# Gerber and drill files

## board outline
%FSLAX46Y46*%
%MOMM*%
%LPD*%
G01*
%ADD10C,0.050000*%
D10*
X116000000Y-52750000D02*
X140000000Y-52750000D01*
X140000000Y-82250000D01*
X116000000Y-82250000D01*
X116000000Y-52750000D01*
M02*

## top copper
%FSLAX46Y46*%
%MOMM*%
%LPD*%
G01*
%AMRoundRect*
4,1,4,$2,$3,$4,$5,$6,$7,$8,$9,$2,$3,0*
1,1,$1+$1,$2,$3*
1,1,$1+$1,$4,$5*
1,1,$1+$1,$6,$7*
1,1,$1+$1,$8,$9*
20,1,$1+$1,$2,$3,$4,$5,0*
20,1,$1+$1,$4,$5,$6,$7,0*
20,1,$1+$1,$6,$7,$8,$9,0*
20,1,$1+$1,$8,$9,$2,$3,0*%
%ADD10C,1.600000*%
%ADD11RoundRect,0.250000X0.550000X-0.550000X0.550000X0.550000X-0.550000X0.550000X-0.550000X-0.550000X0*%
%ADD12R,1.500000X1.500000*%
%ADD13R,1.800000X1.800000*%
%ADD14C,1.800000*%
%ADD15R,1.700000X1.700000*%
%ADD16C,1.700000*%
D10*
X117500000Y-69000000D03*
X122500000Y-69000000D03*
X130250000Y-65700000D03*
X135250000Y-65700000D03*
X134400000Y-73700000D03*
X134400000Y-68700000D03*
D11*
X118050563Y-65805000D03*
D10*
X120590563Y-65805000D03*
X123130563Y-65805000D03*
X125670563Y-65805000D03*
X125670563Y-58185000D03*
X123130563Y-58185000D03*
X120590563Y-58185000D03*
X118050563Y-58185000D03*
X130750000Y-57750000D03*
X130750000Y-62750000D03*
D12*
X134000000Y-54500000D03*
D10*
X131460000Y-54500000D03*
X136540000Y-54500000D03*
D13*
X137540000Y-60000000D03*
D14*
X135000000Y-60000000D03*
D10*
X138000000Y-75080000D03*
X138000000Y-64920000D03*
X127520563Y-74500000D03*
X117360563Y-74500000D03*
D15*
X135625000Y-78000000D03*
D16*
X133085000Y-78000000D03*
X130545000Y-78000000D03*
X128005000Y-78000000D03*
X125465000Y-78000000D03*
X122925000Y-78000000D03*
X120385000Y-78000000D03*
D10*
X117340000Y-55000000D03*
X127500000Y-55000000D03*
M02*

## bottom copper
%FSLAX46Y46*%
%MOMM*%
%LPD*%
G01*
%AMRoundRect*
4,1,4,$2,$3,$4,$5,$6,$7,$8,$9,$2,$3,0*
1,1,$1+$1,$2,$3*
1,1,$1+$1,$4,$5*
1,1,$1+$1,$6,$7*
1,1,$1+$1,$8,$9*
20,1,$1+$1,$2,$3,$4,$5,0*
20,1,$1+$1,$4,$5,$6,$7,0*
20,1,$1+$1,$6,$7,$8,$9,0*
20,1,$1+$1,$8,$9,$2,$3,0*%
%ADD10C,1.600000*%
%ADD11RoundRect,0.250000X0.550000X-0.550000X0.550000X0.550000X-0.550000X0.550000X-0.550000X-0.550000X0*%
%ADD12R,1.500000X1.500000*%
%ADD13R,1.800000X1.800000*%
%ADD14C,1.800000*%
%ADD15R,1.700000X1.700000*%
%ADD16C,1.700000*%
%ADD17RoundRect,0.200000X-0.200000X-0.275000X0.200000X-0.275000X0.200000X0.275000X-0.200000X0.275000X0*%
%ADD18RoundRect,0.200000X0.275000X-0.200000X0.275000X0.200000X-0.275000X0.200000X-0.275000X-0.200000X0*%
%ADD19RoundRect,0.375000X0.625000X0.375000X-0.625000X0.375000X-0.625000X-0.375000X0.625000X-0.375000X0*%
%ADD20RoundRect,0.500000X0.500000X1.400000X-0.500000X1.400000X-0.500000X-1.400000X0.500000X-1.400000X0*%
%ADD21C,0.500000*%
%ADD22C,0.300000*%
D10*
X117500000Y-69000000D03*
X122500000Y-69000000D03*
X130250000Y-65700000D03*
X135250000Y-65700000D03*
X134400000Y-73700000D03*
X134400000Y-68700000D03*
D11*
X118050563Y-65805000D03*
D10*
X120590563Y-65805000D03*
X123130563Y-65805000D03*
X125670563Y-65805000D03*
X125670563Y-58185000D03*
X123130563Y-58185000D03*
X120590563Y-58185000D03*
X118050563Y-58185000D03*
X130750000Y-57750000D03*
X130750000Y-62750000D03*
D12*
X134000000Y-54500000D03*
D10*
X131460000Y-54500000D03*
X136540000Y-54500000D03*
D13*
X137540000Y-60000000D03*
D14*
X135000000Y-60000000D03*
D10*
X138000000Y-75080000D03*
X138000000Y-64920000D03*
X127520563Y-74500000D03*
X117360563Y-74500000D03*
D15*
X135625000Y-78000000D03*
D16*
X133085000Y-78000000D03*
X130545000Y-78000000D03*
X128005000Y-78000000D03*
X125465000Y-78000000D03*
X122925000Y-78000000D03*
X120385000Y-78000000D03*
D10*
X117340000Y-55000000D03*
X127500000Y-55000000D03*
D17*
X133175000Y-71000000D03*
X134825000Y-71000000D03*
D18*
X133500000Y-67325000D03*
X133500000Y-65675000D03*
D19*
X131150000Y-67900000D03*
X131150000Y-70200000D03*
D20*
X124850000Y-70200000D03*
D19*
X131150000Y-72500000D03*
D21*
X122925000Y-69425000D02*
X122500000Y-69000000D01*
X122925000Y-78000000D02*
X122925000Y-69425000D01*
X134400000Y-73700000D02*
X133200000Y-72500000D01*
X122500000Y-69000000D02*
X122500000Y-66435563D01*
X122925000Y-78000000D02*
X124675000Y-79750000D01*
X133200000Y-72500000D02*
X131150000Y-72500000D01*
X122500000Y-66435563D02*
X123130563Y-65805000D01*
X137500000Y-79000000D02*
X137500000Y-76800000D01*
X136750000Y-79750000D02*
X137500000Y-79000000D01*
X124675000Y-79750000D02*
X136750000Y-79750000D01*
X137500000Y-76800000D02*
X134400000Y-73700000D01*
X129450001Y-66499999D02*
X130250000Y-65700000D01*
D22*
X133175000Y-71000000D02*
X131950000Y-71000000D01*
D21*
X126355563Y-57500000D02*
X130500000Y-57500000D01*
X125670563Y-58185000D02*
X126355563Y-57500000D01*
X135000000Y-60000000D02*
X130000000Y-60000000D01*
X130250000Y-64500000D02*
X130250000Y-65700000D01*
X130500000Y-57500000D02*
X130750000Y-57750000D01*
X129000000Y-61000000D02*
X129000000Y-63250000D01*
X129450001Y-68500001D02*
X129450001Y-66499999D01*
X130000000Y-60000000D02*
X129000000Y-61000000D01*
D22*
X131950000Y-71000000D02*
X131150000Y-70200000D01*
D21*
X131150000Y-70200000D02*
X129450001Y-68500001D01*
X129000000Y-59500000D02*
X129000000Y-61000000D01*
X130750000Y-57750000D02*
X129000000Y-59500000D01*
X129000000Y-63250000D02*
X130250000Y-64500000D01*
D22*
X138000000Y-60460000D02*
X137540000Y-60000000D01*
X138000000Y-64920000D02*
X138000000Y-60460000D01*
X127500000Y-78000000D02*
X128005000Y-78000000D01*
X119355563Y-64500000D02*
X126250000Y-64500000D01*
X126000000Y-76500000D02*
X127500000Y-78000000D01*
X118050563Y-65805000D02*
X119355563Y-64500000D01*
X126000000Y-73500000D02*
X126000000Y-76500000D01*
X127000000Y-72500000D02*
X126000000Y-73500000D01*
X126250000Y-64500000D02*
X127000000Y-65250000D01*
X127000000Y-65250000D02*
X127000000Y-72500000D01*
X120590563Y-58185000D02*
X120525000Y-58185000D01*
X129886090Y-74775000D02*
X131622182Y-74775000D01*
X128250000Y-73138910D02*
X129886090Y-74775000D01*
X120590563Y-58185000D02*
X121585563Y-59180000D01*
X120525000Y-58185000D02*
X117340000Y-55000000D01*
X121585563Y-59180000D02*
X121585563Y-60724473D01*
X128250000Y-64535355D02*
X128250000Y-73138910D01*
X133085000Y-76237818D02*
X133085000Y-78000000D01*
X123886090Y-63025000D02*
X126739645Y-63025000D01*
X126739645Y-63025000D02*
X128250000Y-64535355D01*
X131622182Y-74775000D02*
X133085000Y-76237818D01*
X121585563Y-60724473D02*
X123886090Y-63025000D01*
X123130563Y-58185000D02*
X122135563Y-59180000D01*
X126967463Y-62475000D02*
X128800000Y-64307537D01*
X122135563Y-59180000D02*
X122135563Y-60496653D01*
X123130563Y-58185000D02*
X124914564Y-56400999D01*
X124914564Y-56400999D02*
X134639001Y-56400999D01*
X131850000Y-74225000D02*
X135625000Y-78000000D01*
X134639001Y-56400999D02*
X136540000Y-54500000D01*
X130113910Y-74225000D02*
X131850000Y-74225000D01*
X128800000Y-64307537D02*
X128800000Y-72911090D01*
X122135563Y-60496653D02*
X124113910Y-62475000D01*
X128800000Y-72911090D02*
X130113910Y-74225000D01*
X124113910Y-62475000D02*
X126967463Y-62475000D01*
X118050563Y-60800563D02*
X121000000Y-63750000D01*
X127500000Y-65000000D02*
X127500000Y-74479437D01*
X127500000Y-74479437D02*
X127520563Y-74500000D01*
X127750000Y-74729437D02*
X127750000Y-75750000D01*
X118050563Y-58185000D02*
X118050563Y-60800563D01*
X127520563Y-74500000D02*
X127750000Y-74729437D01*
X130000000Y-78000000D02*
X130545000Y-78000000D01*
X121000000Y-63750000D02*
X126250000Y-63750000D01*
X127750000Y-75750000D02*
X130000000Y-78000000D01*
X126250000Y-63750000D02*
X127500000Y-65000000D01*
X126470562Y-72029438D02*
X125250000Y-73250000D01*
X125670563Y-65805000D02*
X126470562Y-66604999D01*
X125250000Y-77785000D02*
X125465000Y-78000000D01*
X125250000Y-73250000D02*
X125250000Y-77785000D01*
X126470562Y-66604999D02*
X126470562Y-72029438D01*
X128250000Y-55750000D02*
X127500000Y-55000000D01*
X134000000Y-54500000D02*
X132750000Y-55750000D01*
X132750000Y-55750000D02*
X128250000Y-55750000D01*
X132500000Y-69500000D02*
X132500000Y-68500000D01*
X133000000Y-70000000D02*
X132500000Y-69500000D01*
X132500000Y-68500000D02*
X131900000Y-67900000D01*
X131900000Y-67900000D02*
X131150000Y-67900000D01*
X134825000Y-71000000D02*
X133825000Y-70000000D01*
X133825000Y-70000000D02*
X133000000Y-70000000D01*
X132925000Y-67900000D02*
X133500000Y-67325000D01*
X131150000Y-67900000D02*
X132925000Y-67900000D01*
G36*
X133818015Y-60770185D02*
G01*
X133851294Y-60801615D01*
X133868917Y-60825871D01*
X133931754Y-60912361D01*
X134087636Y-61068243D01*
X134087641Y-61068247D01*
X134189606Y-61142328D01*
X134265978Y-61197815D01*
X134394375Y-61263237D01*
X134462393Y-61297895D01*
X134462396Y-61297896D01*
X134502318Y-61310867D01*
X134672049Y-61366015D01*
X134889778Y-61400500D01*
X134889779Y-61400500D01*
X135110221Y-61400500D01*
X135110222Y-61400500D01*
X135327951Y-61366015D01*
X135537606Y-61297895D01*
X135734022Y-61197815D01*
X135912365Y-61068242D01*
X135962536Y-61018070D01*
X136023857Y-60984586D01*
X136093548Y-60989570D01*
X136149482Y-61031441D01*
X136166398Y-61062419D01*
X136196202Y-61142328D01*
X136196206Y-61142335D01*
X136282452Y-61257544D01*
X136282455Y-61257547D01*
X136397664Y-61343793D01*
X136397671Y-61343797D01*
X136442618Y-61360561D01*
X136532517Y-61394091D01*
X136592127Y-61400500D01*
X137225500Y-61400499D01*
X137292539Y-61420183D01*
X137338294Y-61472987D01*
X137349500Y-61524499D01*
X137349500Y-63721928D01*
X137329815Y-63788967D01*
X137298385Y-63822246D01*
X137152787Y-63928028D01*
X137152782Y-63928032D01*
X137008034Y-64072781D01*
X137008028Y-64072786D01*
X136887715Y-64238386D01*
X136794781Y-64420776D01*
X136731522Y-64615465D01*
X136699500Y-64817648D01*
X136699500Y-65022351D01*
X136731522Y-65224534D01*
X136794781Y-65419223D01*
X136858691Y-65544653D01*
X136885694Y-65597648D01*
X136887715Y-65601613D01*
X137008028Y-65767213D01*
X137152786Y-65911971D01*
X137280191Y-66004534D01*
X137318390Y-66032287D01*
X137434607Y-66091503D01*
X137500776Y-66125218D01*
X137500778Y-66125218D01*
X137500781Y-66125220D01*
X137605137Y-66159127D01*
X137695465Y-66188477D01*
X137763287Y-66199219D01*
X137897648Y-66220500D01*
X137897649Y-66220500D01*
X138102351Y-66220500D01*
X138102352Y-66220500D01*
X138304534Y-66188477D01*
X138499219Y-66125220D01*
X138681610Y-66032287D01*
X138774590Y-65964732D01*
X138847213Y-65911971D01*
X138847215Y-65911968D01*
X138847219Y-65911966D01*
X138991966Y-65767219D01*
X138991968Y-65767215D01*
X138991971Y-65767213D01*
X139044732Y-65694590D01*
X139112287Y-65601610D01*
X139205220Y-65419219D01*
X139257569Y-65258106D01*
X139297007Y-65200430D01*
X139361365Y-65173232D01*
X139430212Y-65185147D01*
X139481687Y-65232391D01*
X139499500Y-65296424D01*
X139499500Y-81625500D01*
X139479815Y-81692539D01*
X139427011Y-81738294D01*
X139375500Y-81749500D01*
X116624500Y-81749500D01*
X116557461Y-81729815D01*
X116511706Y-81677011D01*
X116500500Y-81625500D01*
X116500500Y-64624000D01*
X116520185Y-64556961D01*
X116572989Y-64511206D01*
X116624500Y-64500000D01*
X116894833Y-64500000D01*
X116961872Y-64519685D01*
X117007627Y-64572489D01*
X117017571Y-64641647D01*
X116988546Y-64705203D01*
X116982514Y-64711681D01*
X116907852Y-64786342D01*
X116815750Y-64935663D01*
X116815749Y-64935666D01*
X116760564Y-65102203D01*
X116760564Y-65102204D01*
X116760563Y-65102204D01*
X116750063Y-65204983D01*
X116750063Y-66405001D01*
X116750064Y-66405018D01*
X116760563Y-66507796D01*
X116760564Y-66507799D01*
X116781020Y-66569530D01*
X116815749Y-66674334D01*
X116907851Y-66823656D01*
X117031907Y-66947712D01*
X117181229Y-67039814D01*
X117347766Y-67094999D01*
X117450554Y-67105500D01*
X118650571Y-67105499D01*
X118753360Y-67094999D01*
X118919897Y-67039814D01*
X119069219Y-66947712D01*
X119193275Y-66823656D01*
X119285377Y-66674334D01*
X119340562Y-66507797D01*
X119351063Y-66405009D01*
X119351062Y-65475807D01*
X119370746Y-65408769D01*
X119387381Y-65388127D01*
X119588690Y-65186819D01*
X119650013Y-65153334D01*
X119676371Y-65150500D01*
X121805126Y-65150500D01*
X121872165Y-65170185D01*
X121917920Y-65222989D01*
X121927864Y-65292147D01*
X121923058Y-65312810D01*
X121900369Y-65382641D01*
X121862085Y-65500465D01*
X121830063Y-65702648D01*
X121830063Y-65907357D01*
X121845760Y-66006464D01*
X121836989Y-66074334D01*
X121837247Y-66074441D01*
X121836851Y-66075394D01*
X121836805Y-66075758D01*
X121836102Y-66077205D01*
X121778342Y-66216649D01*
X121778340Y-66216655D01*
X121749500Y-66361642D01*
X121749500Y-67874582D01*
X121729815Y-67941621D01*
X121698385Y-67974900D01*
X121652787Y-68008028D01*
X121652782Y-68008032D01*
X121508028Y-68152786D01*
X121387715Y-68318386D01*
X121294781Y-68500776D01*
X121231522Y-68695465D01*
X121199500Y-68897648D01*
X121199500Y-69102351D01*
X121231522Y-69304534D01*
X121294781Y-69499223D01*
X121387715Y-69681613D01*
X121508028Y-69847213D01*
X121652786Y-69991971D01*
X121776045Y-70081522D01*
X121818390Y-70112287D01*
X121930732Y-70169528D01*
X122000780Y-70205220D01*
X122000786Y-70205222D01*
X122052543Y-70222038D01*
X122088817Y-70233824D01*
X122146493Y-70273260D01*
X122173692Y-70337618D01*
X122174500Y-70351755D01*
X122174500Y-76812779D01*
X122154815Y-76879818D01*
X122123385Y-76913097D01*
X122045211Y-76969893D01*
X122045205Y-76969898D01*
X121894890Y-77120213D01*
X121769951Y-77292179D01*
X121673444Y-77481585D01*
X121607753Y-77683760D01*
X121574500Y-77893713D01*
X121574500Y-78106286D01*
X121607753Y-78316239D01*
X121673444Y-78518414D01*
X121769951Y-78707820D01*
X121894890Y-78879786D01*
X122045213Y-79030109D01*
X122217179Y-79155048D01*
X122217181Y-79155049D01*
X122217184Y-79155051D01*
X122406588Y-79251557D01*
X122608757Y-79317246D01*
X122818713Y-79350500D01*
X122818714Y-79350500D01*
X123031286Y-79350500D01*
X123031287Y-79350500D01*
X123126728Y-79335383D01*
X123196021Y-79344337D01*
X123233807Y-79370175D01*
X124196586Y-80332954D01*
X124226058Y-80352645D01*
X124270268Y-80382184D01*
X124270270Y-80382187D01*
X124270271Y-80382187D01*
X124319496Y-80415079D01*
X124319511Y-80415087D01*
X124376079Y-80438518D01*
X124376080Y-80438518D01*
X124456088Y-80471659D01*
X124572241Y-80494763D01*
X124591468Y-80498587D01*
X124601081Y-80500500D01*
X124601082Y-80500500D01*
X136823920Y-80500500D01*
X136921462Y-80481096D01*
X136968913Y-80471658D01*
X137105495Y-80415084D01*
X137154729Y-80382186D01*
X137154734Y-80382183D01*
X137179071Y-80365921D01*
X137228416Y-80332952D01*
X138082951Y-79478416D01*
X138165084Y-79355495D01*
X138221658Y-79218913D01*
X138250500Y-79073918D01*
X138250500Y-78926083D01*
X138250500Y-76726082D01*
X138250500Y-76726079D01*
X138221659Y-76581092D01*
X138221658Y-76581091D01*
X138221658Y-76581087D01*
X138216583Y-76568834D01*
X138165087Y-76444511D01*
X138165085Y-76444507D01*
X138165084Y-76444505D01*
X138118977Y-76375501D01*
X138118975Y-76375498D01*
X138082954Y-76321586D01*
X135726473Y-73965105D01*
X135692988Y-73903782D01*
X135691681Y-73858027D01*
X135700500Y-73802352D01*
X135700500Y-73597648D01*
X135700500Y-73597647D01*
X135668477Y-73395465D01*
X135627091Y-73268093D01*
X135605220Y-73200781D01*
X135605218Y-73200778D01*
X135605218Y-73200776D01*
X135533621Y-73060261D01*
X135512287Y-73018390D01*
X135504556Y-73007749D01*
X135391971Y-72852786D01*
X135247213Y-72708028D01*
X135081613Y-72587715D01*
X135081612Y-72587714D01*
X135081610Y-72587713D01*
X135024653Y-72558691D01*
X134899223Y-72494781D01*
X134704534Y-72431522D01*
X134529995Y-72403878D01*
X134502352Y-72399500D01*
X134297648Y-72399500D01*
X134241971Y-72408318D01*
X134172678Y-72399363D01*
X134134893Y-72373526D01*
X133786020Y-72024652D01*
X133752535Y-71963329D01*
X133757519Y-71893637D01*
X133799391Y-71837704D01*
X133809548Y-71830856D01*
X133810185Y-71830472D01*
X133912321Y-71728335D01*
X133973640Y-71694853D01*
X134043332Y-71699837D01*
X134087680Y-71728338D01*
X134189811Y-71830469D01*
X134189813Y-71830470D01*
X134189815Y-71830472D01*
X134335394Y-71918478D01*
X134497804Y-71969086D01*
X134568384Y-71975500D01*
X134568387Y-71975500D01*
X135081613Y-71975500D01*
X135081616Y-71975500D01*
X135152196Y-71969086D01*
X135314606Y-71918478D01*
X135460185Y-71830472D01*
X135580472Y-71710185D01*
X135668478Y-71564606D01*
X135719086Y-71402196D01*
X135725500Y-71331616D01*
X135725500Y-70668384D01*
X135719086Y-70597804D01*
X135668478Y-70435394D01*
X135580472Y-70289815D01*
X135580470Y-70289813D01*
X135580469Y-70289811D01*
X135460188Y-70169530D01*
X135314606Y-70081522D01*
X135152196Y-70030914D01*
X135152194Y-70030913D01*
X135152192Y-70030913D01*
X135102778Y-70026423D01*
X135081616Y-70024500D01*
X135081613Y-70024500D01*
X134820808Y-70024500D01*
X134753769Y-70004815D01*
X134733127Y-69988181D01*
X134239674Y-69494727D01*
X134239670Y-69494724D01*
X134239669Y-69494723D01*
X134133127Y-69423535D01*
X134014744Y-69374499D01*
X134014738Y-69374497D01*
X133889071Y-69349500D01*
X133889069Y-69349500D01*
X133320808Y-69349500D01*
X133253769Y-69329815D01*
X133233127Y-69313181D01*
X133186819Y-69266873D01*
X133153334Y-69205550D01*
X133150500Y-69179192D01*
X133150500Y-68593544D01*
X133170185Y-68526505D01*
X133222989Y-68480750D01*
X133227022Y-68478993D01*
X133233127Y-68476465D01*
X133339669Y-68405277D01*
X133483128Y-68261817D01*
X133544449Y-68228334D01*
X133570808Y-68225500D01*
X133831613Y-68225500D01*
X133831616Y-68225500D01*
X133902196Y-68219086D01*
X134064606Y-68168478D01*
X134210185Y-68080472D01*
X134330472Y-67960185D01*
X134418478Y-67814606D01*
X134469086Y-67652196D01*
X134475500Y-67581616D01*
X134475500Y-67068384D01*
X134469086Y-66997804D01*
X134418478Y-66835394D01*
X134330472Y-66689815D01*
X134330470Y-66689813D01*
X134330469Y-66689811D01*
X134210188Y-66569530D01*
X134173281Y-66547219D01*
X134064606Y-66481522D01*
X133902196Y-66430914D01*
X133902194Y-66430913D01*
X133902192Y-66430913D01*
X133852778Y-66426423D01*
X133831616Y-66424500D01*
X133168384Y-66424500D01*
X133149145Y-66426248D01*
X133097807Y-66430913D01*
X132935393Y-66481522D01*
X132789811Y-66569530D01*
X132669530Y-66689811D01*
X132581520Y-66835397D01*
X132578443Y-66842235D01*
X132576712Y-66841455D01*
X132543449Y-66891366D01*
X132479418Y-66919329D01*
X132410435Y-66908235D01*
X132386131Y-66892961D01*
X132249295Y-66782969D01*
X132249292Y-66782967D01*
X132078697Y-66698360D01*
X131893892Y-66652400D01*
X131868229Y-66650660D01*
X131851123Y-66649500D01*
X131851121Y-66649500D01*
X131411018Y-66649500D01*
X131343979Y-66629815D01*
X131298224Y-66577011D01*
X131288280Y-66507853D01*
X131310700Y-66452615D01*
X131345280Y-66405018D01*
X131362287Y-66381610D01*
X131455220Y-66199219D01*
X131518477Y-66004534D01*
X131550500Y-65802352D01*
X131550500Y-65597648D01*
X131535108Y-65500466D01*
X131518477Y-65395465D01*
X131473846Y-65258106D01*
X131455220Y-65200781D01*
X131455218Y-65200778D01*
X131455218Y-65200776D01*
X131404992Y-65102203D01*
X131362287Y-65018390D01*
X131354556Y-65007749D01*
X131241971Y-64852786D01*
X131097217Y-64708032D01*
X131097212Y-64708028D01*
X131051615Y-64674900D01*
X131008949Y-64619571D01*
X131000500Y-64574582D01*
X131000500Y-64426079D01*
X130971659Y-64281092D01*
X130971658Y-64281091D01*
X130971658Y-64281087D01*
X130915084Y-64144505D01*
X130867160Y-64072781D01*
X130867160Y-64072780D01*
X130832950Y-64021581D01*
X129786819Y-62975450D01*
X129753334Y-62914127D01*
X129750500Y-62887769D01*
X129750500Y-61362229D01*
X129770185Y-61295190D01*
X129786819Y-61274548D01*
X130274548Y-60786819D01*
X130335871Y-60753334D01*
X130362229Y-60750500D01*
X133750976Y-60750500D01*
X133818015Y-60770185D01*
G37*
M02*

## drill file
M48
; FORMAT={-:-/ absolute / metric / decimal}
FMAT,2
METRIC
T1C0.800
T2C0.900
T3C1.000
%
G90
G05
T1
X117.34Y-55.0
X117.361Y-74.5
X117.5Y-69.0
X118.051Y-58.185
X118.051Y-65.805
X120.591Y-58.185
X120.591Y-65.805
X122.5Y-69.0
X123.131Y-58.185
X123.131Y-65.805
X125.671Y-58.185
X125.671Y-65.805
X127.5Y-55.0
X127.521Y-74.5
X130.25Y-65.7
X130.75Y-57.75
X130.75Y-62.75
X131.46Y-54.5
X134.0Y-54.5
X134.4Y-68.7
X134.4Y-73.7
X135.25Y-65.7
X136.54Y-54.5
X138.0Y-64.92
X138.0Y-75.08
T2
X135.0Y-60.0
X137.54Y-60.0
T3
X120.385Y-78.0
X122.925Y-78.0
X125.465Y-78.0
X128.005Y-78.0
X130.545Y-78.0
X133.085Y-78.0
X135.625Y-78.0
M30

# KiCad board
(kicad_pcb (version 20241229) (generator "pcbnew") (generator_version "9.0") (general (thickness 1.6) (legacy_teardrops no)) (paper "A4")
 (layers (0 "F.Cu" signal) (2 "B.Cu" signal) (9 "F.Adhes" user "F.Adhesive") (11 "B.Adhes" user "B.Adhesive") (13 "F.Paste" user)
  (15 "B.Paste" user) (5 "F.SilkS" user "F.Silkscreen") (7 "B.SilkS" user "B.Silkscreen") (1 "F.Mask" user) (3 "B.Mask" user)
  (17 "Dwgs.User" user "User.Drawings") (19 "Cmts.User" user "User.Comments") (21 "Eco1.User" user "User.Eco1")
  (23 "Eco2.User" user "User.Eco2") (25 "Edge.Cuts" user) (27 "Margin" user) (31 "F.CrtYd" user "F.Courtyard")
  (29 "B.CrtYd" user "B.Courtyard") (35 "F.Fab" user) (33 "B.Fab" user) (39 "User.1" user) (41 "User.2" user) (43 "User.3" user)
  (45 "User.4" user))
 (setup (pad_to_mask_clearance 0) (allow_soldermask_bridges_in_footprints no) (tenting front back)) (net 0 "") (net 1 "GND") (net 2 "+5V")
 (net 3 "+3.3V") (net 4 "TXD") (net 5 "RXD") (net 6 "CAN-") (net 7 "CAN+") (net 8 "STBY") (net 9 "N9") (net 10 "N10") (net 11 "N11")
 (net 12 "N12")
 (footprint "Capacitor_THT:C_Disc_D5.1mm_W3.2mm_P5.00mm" (layer "F.Cu") (at 117.5 69)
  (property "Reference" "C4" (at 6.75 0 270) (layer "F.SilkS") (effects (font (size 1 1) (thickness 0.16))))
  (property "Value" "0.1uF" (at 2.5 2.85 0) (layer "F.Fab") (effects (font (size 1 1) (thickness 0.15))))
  (pad "1" thru_hole circle (at 0 0) (size 1.6 1.6) (drill 0.8) (layers "*.Cu" "*.Mask") (remove_unused_layers no) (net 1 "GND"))
  (pad "2" thru_hole circle (at 5 0) (size 1.6 1.6) (drill 0.8) (layers "*.Cu" "*.Mask") (remove_unused_layers no) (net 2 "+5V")))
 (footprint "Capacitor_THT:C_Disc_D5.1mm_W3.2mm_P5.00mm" (layer "F.Cu") (at 130.25 65.7)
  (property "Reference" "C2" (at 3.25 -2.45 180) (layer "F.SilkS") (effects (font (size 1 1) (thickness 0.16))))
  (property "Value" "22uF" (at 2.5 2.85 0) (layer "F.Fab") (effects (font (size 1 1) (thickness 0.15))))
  (pad "1" thru_hole circle (at 0 0) (size 1.6 1.6) (drill 0.8) (layers "*.Cu" "*.Mask") (remove_unused_layers no) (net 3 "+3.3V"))
  (pad "2" thru_hole circle (at 5 0) (size 1.6 1.6) (drill 0.8) (layers "*.Cu" "*.Mask") (remove_unused_layers no) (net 1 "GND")))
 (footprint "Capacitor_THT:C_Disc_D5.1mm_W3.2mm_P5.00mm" (layer "F.Cu") (at 134.4 73.7 90)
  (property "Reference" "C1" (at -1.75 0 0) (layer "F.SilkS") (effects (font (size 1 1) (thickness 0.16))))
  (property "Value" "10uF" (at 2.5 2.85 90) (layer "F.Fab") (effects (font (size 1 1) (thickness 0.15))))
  (pad "1" thru_hole circle (at 0 0 90) (size 1.6 1.6) (drill 0.8) (layers "*.Cu" "*.Mask") (remove_unused_layers no) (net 2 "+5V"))
  (pad "2" thru_hole circle (at 5 0 90) (size 1.6 1.6) (drill 0.8) (layers "*.Cu" "*.Mask") (remove_unused_layers no) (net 1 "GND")))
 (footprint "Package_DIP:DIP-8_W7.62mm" (layer "F.Cu") (at 118.050563 65.805 90)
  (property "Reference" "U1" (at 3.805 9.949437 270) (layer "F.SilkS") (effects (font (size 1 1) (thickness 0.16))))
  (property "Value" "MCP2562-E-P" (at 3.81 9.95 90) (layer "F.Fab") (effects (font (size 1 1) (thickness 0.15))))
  (pad "1" thru_hole roundrect (at 0 0 90) (size 1.6 1.6) (drill 0.8) (layers "*.Cu" "*.Mask") (remove_unused_layers no)
   (roundrect_rratio 0.15625) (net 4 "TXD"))
  (pad "2" thru_hole circle (at 0 2.54 90) (size 1.6 1.6) (drill 0.8) (layers "*.Cu" "*.Mask") (remove_unused_layers no) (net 1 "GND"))
  (pad "3" thru_hole circle (at 0 5.08 90) (size 1.6 1.6) (drill 0.8) (layers "*.Cu" "*.Mask") (remove_unused_layers no) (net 2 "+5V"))
  (pad "4" thru_hole circle (at 0 7.62 90) (size 1.6 1.6) (drill 0.8) (layers "*.Cu" "*.Mask") (remove_unused_layers no) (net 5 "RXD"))
  (pad "5" thru_hole circle (at 7.62 7.62 90) (size 1.6 1.6) (drill 0.8) (layers "*.Cu" "*.Mask") (remove_unused_layers no) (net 3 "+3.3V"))
  (pad "6" thru_hole circle (at 7.62 5.08 90) (size 1.6 1.6) (drill 0.8) (layers "*.Cu" "*.Mask") (remove_unused_layers no) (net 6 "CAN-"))
  (pad "7" thru_hole circle (at 7.62 2.54 90) (size 1.6 1.6) (drill 0.8) (layers "*.Cu" "*.Mask") (remove_unused_layers no) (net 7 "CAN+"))
  (pad "8" thru_hole circle (at 7.62 0 90) (size 1.6 1.6) (drill 0.8) (layers "*.Cu" "*.Mask") (remove_unused_layers no) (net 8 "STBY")))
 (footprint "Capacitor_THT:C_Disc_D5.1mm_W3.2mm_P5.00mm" (layer "F.Cu") (at 130.75 57.75 -90)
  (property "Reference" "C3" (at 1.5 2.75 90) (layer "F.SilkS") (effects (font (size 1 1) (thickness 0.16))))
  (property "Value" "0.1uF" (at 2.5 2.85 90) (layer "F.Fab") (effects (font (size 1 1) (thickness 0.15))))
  (pad "1" thru_hole circle (at 0 0 270) (size 1.6 1.6) (drill 0.8) (layers "*.Cu" "*.Mask") (remove_unused_layers no) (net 3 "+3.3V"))
  (pad "2" thru_hole circle (at 5 0 270) (size 1.6 1.6) (drill 0.8) (layers "*.Cu" "*.Mask") (remove_unused_layers no) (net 1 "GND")))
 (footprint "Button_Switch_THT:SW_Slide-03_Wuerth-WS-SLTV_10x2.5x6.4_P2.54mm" (layer "F.Cu") (at 134 54.5)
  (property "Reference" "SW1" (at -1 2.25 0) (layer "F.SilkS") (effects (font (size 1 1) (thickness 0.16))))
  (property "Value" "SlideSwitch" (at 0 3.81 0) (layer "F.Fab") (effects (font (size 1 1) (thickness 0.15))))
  (pad "1" thru_hole rect (at 0 0) (size 1.5 1.5) (drill 0.8) (layers "*.Cu" "*.Mask") (remove_unused_layers no) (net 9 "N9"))
  (pad "2" thru_hole circle (at -2.54 0) (size 1.6 1.6) (drill 0.8) (layers "*.Cu" "*.Mask") (remove_unused_layers no) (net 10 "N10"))
  (pad "3" thru_hole circle (at 2.54 0) (size 1.6 1.6) (drill 0.8) (layers "*.Cu" "*.Mask") (remove_unused_layers no) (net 6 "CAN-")))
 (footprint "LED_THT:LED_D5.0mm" (layer "F.Cu") (at 137.54 60 180)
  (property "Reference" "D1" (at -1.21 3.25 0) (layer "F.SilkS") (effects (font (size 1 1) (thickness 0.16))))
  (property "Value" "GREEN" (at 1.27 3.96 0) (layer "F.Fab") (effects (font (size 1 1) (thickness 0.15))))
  (pad "1" thru_hole rect (at 0 0 180) (size 1.8 1.8) (drill 0.9) (layers "*.Cu" "*.Mask") (remove_unused_layers no) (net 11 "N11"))
  (pad "2" thru_hole circle (at 2.54 0 180) (size 1.8 1.8) (drill 0.9) (layers "*.Cu" "*.Mask") (remove_unused_layers no) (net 3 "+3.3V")))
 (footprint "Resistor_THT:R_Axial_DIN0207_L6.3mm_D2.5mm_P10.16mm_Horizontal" (layer "F.Cu") (at 138 75.08 90)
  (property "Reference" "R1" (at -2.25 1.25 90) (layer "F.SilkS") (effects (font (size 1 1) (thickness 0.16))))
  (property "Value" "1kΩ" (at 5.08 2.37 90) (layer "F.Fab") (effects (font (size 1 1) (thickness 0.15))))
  (pad "1" thru_hole circle (at 0 0 90) (size 1.6 1.6) (drill 0.8) (layers "*.Cu" "*.Mask") (remove_unused_layers no) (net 1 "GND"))
  (pad "2" thru_hole circle (at 10.16 0 90) (size 1.6 1.6) (drill 0.8) (layers "*.Cu" "*.Mask") (remove_unused_layers no) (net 11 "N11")))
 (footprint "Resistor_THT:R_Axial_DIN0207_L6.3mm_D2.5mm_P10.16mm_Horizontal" (layer "F.Cu") (at 127.520563 74.5 180)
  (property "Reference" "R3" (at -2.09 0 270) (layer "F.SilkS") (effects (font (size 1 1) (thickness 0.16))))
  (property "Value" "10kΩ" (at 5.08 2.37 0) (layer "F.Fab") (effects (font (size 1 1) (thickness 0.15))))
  (pad "1" thru_hole circle (at 0 0 180) (size 1.6 1.6) (drill 0.8) (layers "*.Cu" "*.Mask") (remove_unused_layers no) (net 8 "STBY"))
  (pad "2" thru_hole circle (at 10.16 0 180) (size 1.6 1.6) (drill 0.8) (layers "*.Cu" "*.Mask") (remove_unused_layers no) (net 1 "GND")))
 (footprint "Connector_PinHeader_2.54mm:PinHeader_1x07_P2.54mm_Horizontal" (layer "F.Cu") (at 135.625 78 -90)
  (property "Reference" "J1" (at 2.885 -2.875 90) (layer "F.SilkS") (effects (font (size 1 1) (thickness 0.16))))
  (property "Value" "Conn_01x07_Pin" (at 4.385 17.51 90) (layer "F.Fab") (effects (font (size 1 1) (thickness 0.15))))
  (pad "1" thru_hole rect (at 0 0 270) (size 1.7 1.7) (drill 1) (layers "*.Cu" "*.Mask") (remove_unused_layers no) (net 6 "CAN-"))
  (pad "2" thru_hole circle (at 0 2.54 270) (size 1.7 1.7) (drill 1) (layers "*.Cu" "*.Mask") (remove_unused_layers no) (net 7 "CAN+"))
  (pad "3" thru_hole circle (at 0 5.08 270) (size 1.7 1.7) (drill 1) (layers "*.Cu" "*.Mask") (remove_unused_layers no) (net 8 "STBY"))
  (pad "4" thru_hole circle (at 0 7.62 270) (size 1.7 1.7) (drill 1) (layers "*.Cu" "*.Mask") (remove_unused_layers no) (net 4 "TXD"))
  (pad "5" thru_hole circle (at 0 10.16 270) (size 1.7 1.7) (drill 1) (layers "*.Cu" "*.Mask") (remove_unused_layers no) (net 5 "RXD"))
  (pad "6" thru_hole circle (at 0 12.7 270) (size 1.7 1.7) (drill 1) (layers "*.Cu" "*.Mask") (remove_unused_layers no) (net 2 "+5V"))
  (pad "7" thru_hole circle (at 0 15.24 270) (size 1.7 1.7) (drill 1) (layers "*.Cu" "*.Mask") (remove_unused_layers no) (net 1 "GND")))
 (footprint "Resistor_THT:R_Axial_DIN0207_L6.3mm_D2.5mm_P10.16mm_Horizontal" (layer "F.Cu") (at 117.34 55)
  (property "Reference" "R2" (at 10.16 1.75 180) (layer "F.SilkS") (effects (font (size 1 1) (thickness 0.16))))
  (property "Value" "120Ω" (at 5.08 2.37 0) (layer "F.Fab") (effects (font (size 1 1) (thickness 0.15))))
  (pad "1" thru_hole circle (at 0 0) (size 1.6 1.6) (drill 0.8) (layers "*.Cu" "*.Mask") (remove_unused_layers no) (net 7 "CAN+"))
  (pad "2" thru_hole circle (at 10.16 0) (size 1.6 1.6) (drill 0.8) (layers "*.Cu" "*.Mask") (remove_unused_layers no) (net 9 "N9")))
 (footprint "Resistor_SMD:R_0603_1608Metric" (layer "B.Cu") (at 134 71)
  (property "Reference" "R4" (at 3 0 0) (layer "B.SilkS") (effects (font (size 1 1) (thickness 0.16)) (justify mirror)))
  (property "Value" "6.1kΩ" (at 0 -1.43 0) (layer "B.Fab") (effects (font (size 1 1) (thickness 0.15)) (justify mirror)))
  (pad "1" smd roundrect (at -0.825 0) (size 0.8 0.95) (layers "B.Cu" "B.Mask" "B.Paste") (roundrect_rratio 0.25) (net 3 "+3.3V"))
  (pad "2" smd roundrect (at 0.825 0) (size 0.8 0.95) (layers "B.Cu" "B.Mask" "B.Paste") (roundrect_rratio 0.25) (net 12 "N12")))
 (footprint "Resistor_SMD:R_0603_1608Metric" (layer "B.Cu") (at 133.5 66.5 90)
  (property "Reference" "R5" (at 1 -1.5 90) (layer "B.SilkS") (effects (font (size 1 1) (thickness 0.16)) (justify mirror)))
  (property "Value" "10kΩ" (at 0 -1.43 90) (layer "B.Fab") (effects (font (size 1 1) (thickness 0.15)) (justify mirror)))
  (pad "1" smd roundrect (at -0.825 0 90) (size 0.8 0.95) (layers "B.Cu" "B.Mask" "B.Paste") (roundrect_rratio 0.25) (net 12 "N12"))
  (pad "2" smd roundrect (at 0.825 0 90) (size 0.8 0.95) (layers "B.Cu" "B.Mask" "B.Paste") (roundrect_rratio 0.25) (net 1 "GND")))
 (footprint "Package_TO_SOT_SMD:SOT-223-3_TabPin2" (layer "B.Cu") (at 128 70.2 180)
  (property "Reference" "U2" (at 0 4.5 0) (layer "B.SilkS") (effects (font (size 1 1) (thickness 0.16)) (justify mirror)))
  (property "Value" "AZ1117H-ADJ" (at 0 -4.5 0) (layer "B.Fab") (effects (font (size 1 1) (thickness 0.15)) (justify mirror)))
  (pad "1" smd roundrect (at -3.15 2.3 180) (size 2 1.5) (layers "B.Cu" "B.Mask" "B.Paste") (roundrect_rratio 0.25) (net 12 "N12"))
  (pad "2" smd roundrect (at -3.15 0 180) (size 2 1.5) (layers "B.Cu" "B.Mask" "B.Paste") (roundrect_rratio 0.25) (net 3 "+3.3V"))
  (pad "2" smd roundrect (at 3.15 0 180) (size 2 3.8) (layers "B.Cu" "B.Mask" "B.Paste") (roundrect_rratio 0.25) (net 3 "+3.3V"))
  (pad "3" smd roundrect (at -3.15 -2.3 180) (size 2 1.5) (layers "B.Cu" "B.Mask" "B.Paste") (roundrect_rratio 0.25) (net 2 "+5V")))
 (gr_rect (start 116 52.75) (end 140 82.25) (stroke (width 0.05) (type default)) (fill no) (layer "Edge.Cuts"))
 (segment (start 122.925 69.425) (end 122.5 69) (width 0.5) (layer "B.Cu") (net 2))
 (segment (start 122.925 78) (end 122.925 69.425) (width 0.5) (layer "B.Cu") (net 2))
 (segment (start 134.4 73.7) (end 133.2 72.5) (width 0.5) (layer "B.Cu") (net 2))
 (segment (start 122.5 69) (end 122.5 66.435563) (width 0.5) (layer "B.Cu") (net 2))
 (segment (start 122.925 78) (end 124.675 79.75) (width 0.5) (layer "B.Cu") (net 2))
 (segment (start 133.2 72.5) (end 131.15 72.5) (width 0.5) (layer "B.Cu") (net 2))
 (segment (start 122.5 66.435563) (end 123.130563 65.805) (width 0.5) (layer "B.Cu") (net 2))
 (segment (start 137.5 79) (end 137.5 76.8) (width 0.5) (layer "B.Cu") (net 2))
 (segment (start 136.75 79.75) (end 137.5 79) (width 0.5) (layer "B.Cu") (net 2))
 (segment (start 124.675 79.75) (end 136.75 79.75) (width 0.5) (layer "B.Cu") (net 2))
 (segment (start 137.5 76.8) (end 134.4 73.7) (width 0.5) (layer "B.Cu") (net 2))
 (segment (start 129.450001 66.499999) (end 130.25 65.7) (width 0.5) (layer "B.Cu") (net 3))
 (segment (start 133.175 71) (end 131.95 71) (width 0.3) (layer "B.Cu") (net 3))
 (segment (start 126.355563 57.5) (end 130.5 57.5) (width 0.5) (layer "B.Cu") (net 3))
 (segment (start 125.670563 58.185) (end 126.355563 57.5) (width 0.5) (layer "B.Cu") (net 3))
 (segment (start 135 60) (end 130 60) (width 0.5) (layer "B.Cu") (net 3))
 (segment (start 130.25 64.5) (end 130.25 65.7) (width 0.5) (layer "B.Cu") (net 3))
 (segment (start 130.5 57.5) (end 130.75 57.75) (width 0.5) (layer "B.Cu") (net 3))
 (segment (start 129 61) (end 129 63.25) (width 0.5) (layer "B.Cu") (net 3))
 (segment (start 129.450001 68.500001) (end 129.450001 66.499999) (width 0.5) (layer "B.Cu") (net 3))
 (segment (start 130 60) (end 129 61) (width 0.5) (layer "B.Cu") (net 3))
 (segment (start 131.95 71) (end 131.15 70.2) (width 0.3) (layer "B.Cu") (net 3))
 (segment (start 131.15 70.2) (end 129.450001 68.500001) (width 0.5) (layer "B.Cu") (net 3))
 (segment (start 129 59.5) (end 129 61) (width 0.5) (layer "B.Cu") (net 3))
 (segment (start 130.75 57.75) (end 129 59.5) (width 0.5) (layer "B.Cu") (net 3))
 (segment (start 129 63.25) (end 130.25 64.5) (width 0.5) (layer "B.Cu") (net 3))
 (segment (start 138 60.46) (end 137.54 60) (width 0.3) (layer "B.Cu") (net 11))
 (segment (start 138 64.92) (end 138 60.46) (width 0.3) (layer "B.Cu") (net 11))
 (segment (start 127.5 78) (end 128.005 78) (width 0.3) (layer "B.Cu") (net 4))
 (segment (start 119.355563 64.5) (end 126.25 64.5) (width 0.3) (layer "B.Cu") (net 4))
 (segment (start 126 76.5) (end 127.5 78) (width 0.3) (layer "B.Cu") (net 4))
 (segment (start 118.050563 65.805) (end 119.355563 64.5) (width 0.3) (layer "B.Cu") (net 4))
 (segment (start 126 73.5) (end 126 76.5) (width 0.3) (layer "B.Cu") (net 4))
 (segment (start 127 72.5) (end 126 73.5) (width 0.3) (layer "B.Cu") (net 4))
 (segment (start 126.25 64.5) (end 127 65.25) (width 0.3) (layer "B.Cu") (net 4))
 (segment (start 127 65.25) (end 127 72.5) (width 0.3) (layer "B.Cu") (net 4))
 (segment (start 120.590563 58.185) (end 120.525 58.185) (width 0.3) (layer "B.Cu") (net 7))
 (segment (start 129.88609 74.775) (end 131.622182 74.775) (width 0.3) (layer "B.Cu") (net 7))
 (segment (start 128.25 73.13891) (end 129.88609 74.775) (width 0.3) (layer "B.Cu") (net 7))
 (segment (start 120.590563 58.185) (end 121.585563 59.18) (width 0.3) (layer "B.Cu") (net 7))
 (segment (start 120.525 58.185) (end 117.34 55) (width 0.3) (layer "B.Cu") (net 7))
 (segment (start 121.585563 59.18) (end 121.585563 60.724473) (width 0.3) (layer "B.Cu") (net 7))
 (segment (start 128.25 64.535355) (end 128.25 73.13891) (width 0.3) (layer "B.Cu") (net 7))
 (segment (start 133.085 76.237818) (end 133.085 78) (width 0.3) (layer "B.Cu") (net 7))
 (segment (start 123.88609 63.025) (end 126.739645 63.025) (width 0.3) (layer "B.Cu") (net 7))
 (segment (start 126.739645 63.025) (end 128.25 64.535355) (width 0.3) (layer "B.Cu") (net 7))
 (segment (start 131.622182 74.775) (end 133.085 76.237818) (width 0.3) (layer "B.Cu") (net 7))
 (segment (start 121.585563 60.724473) (end 123.88609 63.025) (width 0.3) (layer "B.Cu") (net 7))
 (segment (start 123.130563 58.185) (end 122.135563 59.18) (width 0.3) (layer "B.Cu") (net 6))
 (segment (start 126.967463 62.475) (end 128.8 64.307537) (width 0.3) (layer "B.Cu") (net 6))
 (segment (start 122.135563 59.18) (end 122.135563 60.496653) (width 0.3) (layer "B.Cu") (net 6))
 (segment (start 123.130563 58.185) (end 124.914564 56.400999) (width 0.3) (layer "B.Cu") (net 6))
 (segment (start 124.914564 56.400999) (end 134.639001 56.400999) (width 0.3) (layer "B.Cu") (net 6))
 (segment (start 131.85 74.225) (end 135.625 78) (width 0.3) (layer "B.Cu") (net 6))
 (segment (start 134.639001 56.400999) (end 136.54 54.5) (width 0.3) (layer "B.Cu") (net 6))
 (segment (start 130.11391 74.225) (end 131.85 74.225) (width 0.3) (layer "B.Cu") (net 6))
 (segment (start 128.8 64.307537) (end 128.8 72.91109) (width 0.3) (layer "B.Cu") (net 6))
 (segment (start 122.135563 60.496653) (end 124.11391 62.475) (width 0.3) (layer "B.Cu") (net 6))
 (segment (start 128.8 72.91109) (end 130.11391 74.225) (width 0.3) (layer "B.Cu") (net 6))
 (segment (start 124.11391 62.475) (end 126.967463 62.475) (width 0.3) (layer "B.Cu") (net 6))
 (segment (start 118.050563 60.800563) (end 121 63.75) (width 0.3) (layer "B.Cu") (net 8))
 (segment (start 127.5 65) (end 127.5 74.479437) (width 0.3) (layer "B.Cu") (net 8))
 (segment (start 127.5 74.479437) (end 127.520563 74.5) (width 0.3) (layer "B.Cu") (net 8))
 (segment (start 127.75 74.729437) (end 127.75 75.75) (width 0.3) (layer "B.Cu") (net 8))
 (segment (start 118.050563 58.185) (end 118.050563 60.800563) (width 0.3) (layer "B.Cu") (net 8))
 (segment (start 127.520563 74.5) (end 127.75 74.729437) (width 0.3) (layer "B.Cu") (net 8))
 (segment (start 130 78) (end 130.545 78) (width 0.3) (layer "B.Cu") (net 8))
 (segment (start 121 63.75) (end 126.25 63.75) (width 0.3) (layer "B.Cu") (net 8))
 (segment (start 127.75 75.75) (end 130 78) (width 0.3) (layer "B.Cu") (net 8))
 (segment (start 126.25 63.75) (end 127.5 65) (width 0.3) (layer "B.Cu") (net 8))
 (segment (start 126.470562 72.029438) (end 125.25 73.25) (width 0.3) (layer "B.Cu") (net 5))
 (segment (start 125.670563 65.805) (end 126.470562 66.604999) (width 0.3) (layer "B.Cu") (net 5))
 (segment (start 125.25 77.785) (end 125.465 78) (width 0.3) (layer "B.Cu") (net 5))
 (segment (start 125.25 73.25) (end 125.25 77.785) (width 0.3) (layer "B.Cu") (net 5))
 (segment (start 126.470562 66.604999) (end 126.470562 72.029438) (width 0.3) (layer "B.Cu") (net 5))
 (segment (start 128.25 55.75) (end 127.5 55) (width 0.3) (layer "B.Cu") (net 9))
 (segment (start 134 54.5) (end 132.75 55.75) (width 0.3) (layer "B.Cu") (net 9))
 (segment (start 132.75 55.75) (end 128.25 55.75) (width 0.3) (layer "B.Cu") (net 9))
 (segment (start 132.5 69.5) (end 132.5 68.5) (width 0.3) (layer "B.Cu") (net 12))
 (segment (start 133 70) (end 132.5 69.5) (width 0.3) (layer "B.Cu") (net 12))
 (segment (start 132.5 68.5) (end 131.9 67.9) (width 0.3) (layer "B.Cu") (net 12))
 (segment (start 131.9 67.9) (end 131.15 67.9) (width 0.3) (layer "B.Cu") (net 12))
 (segment (start 134.825 71) (end 133.825 70) (width 0.3) (layer "B.Cu") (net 12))
 (segment (start 133.825 70) (end 133 70) (width 0.3) (layer "B.Cu") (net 12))
 (segment (start 132.925 67.9) (end 133.5 67.325) (width 0.3) (layer "B.Cu") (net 12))
 (segment (start 131.15 67.9) (end 132.925 67.9) (width 0.3) (layer "B.Cu") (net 12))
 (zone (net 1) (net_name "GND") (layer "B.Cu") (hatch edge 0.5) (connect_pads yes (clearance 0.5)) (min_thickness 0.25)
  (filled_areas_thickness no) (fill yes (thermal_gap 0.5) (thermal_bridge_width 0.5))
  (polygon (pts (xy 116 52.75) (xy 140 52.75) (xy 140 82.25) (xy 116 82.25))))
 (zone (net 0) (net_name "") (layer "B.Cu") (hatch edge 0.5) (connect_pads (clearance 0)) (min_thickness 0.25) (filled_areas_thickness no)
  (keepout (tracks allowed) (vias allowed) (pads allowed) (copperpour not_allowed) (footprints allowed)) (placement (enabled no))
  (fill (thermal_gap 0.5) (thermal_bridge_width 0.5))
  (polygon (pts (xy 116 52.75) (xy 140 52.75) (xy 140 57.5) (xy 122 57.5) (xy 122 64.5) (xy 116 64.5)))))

